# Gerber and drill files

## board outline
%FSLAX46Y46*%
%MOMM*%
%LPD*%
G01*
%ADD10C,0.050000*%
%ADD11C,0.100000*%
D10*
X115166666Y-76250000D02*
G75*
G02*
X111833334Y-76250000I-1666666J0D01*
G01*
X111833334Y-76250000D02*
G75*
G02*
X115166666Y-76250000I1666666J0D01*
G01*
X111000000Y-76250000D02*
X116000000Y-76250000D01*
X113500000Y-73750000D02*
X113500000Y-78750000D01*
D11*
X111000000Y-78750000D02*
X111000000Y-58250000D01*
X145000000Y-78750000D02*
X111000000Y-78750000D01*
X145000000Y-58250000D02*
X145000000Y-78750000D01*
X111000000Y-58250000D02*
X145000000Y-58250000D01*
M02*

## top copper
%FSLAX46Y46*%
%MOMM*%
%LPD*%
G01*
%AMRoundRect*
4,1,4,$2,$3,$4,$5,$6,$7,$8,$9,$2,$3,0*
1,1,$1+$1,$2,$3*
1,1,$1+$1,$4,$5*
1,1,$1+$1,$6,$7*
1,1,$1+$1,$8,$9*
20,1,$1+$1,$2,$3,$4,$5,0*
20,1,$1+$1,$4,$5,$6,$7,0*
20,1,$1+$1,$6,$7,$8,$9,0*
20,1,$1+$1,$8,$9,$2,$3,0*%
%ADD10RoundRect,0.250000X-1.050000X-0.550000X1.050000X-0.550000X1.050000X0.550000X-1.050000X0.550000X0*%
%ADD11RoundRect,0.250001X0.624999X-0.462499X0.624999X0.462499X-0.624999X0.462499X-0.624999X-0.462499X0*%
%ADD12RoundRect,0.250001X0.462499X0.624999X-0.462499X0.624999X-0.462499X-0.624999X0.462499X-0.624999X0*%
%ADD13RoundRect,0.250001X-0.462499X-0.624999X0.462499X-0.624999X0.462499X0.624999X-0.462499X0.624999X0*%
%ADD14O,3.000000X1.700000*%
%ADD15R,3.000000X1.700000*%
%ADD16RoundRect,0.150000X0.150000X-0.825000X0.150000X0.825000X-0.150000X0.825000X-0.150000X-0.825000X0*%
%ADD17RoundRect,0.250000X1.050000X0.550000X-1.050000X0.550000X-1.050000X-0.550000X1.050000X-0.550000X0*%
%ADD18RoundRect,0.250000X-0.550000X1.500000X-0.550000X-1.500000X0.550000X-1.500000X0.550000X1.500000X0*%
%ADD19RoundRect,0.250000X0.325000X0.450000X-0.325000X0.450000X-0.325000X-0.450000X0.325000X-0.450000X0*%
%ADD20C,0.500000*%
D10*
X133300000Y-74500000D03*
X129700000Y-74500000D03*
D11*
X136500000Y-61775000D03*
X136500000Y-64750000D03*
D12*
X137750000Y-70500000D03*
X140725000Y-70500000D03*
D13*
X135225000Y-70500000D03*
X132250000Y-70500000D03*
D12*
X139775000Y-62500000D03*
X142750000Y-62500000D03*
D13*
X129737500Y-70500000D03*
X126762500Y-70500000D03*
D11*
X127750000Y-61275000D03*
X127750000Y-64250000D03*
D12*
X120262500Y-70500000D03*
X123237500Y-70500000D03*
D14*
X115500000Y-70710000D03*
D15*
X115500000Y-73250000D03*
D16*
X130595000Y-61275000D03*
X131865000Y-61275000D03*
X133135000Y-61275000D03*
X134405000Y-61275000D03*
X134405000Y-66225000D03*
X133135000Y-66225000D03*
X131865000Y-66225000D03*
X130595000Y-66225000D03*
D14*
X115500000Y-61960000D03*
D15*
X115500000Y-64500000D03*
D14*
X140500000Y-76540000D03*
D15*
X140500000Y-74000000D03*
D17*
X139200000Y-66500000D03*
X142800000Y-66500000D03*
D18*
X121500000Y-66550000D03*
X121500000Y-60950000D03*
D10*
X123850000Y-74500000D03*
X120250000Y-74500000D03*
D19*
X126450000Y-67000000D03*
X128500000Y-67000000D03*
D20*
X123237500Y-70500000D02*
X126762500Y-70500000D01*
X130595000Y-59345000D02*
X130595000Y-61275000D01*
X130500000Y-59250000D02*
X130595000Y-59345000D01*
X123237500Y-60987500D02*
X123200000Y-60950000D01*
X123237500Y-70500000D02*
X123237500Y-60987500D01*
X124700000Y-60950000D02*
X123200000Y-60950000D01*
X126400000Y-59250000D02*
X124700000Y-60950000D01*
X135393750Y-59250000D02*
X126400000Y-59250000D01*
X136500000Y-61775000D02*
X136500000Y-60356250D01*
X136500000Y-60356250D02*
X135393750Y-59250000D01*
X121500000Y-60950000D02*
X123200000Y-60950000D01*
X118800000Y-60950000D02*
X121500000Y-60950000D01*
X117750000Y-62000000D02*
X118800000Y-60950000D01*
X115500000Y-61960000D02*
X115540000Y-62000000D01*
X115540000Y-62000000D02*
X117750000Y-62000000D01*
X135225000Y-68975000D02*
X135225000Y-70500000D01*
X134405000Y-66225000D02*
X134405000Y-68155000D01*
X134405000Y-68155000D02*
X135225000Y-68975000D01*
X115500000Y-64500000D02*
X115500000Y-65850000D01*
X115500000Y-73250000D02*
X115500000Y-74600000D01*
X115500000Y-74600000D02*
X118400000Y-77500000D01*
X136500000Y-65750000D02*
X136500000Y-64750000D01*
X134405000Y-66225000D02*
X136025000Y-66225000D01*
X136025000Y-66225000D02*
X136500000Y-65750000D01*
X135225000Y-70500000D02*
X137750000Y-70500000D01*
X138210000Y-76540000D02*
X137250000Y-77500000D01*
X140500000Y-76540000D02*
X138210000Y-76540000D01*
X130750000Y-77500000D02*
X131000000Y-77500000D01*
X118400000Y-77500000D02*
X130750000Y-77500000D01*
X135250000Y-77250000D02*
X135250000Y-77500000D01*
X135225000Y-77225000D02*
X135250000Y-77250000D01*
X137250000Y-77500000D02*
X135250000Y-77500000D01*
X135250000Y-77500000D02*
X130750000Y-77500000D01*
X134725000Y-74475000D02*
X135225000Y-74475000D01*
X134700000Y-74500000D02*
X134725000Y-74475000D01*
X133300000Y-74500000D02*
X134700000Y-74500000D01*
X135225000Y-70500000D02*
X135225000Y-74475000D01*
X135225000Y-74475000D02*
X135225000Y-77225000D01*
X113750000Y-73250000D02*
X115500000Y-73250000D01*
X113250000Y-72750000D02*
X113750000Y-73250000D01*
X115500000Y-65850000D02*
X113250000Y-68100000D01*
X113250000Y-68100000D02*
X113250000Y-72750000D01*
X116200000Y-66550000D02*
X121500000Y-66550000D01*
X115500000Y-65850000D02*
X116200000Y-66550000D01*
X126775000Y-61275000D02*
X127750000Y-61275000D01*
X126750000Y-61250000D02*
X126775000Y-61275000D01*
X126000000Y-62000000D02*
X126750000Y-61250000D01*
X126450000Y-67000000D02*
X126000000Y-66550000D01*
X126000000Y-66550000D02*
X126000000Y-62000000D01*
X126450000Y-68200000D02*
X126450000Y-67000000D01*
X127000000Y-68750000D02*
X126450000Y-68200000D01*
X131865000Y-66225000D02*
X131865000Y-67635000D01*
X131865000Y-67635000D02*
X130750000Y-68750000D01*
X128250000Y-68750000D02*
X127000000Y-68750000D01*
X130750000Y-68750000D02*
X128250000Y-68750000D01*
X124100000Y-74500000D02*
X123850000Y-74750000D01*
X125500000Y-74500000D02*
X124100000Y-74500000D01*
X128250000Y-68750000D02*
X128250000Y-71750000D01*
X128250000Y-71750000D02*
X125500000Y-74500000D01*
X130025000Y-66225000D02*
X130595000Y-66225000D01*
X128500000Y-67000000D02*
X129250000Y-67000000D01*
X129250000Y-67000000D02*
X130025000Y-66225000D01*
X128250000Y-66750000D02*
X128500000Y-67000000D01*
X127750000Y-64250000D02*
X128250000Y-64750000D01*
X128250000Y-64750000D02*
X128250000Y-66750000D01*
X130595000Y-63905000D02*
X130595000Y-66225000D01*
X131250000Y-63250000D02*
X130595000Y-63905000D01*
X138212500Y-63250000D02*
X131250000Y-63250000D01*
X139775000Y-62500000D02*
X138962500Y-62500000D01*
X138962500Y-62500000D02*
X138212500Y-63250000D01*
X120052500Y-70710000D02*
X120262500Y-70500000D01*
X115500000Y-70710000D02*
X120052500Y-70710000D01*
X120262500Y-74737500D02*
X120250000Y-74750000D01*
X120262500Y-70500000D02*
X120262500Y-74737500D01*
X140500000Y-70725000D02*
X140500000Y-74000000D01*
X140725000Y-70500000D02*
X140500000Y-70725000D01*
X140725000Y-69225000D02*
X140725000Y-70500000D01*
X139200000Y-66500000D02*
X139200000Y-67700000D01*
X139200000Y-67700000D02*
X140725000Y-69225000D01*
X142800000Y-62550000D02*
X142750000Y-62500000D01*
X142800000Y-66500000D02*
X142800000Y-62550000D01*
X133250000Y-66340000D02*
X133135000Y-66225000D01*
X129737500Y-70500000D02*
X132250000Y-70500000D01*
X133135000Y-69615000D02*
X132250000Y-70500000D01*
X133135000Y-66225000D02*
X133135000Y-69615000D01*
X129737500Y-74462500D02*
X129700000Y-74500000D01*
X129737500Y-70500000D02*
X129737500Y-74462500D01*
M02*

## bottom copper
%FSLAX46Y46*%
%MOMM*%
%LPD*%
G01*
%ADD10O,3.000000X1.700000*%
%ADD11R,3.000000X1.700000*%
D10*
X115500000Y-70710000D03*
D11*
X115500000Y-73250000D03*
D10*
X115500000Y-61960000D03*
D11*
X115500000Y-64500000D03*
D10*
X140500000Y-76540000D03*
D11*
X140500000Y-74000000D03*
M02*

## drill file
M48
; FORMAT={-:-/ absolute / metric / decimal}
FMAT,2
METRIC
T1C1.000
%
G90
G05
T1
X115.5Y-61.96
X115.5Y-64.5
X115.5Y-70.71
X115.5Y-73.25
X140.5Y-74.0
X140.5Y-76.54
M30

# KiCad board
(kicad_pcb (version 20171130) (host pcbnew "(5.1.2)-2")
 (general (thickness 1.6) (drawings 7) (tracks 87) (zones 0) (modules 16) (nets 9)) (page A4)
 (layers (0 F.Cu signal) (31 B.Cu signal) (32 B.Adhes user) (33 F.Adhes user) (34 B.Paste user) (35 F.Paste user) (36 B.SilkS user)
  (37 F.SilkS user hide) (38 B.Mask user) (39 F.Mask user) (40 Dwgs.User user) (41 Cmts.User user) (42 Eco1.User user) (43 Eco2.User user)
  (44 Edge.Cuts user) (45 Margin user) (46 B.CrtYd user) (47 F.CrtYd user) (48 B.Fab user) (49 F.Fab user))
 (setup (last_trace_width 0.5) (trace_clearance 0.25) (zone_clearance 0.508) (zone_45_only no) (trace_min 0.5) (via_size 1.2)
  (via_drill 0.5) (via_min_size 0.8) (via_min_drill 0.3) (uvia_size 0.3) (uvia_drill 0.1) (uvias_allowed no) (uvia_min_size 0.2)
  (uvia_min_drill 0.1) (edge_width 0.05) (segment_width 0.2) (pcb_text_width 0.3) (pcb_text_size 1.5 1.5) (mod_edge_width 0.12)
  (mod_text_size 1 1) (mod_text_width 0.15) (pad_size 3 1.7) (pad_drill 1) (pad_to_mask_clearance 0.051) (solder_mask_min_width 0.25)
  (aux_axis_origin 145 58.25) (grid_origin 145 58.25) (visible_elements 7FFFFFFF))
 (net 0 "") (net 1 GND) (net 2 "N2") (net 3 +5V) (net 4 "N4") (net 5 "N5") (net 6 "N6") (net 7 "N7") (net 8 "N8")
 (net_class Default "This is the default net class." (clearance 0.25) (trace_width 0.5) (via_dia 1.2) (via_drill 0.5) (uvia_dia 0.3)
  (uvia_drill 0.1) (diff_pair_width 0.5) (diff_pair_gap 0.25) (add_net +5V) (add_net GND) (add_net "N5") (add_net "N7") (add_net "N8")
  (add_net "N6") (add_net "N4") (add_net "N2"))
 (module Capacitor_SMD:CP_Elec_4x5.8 (layer F.Cu) (at 131.5 74.5)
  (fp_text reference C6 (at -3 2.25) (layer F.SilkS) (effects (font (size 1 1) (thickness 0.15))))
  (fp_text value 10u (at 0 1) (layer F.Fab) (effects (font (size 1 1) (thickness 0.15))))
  (pad 2 smd roundrect (at 1.8 0) (size 2.6 1.6) (layers F.Cu F.Paste F.Mask) (roundrect_rratio 0.15625) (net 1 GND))
  (pad 1 smd roundrect (at -1.8 0) (size 2.6 1.6) (layers F.Cu F.Paste F.Mask) (roundrect_rratio 0.15625) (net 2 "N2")))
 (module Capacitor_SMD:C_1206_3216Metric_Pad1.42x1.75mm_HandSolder (layer F.Cu) (at 136.5 63.2625 90)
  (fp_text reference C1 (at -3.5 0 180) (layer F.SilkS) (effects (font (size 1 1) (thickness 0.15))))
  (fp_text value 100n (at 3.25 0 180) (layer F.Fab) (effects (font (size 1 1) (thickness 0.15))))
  (pad 2 smd roundrect (at 1.4875 0 90) (size 1.425 1.75) (layers F.Cu F.Paste F.Mask) (roundrect_rratio 0.175439) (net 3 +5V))
  (pad 1 smd roundrect (at -1.4875 0 90) (size 1.425 1.75) (layers F.Cu F.Paste F.Mask) (roundrect_rratio 0.175439) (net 1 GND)))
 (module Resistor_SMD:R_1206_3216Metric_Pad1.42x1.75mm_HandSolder (layer F.Cu) (at 139.2375 70.5 180)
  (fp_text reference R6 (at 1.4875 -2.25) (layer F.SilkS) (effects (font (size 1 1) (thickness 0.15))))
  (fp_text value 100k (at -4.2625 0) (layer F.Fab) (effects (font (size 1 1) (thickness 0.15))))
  (pad 2 smd roundrect (at 1.4875 0 180) (size 1.425 1.75) (layers F.Cu F.Paste F.Mask) (roundrect_rratio 0.175439) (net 1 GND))
  (pad 1 smd roundrect (at -1.4875 0 180) (size 1.425 1.75) (layers F.Cu F.Paste F.Mask) (roundrect_rratio 0.175439) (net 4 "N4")))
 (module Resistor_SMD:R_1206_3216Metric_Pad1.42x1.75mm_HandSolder (layer F.Cu) (at 133.7375 70.5)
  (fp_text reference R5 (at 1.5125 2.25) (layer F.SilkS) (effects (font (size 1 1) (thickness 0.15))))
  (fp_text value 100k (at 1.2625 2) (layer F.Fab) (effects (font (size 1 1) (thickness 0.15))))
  (pad 2 smd roundrect (at 1.4875 0) (size 1.425 1.75) (layers F.Cu F.Paste F.Mask) (roundrect_rratio 0.175439) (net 1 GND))
  (pad 1 smd roundrect (at -1.4875 0) (size 1.425 1.75) (layers F.Cu F.Paste F.Mask) (roundrect_rratio 0.175439) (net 2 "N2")))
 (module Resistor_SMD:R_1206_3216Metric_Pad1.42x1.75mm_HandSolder (layer F.Cu) (at 141.2625 62.5 180)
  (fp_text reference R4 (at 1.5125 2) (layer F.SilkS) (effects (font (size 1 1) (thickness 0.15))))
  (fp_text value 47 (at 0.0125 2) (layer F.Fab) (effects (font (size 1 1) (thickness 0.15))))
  (pad 2 smd roundrect (at 1.4875 0 180) (size 1.425 1.75) (layers F.Cu F.Paste F.Mask) (roundrect_rratio 0.175439) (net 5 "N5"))
  (pad 1 smd roundrect (at -1.4875 0 180) (size 1.425 1.75) (layers F.Cu F.Paste F.Mask) (roundrect_rratio 0.175439) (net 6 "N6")))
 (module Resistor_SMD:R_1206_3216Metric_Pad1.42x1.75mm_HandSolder (layer F.Cu) (at 128.25 70.5)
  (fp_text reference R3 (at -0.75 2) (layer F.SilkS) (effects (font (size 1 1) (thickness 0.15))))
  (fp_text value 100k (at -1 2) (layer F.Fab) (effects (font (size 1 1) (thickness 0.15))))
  (pad 2 smd roundrect (at 1.4875 0) (size 1.425 1.75) (layers F.Cu F.Paste F.Mask) (roundrect_rratio 0.175439) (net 2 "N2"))
  (pad 1 smd roundrect (at -1.4875 0) (size 1.425 1.75) (layers F.Cu F.Paste F.Mask) (roundrect_rratio 0.175439) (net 3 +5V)))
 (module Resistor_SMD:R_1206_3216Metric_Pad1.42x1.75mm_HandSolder (layer F.Cu) (at 127.75 62.7625 90)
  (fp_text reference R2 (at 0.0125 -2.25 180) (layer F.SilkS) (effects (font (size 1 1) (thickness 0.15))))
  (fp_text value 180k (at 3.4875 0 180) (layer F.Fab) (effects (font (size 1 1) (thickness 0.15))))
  (pad 2 smd roundrect (at 1.4875 0 90) (size 1.425 1.75) (layers F.Cu F.Paste F.Mask) (roundrect_rratio 0.175439) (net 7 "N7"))
  (pad 1 smd roundrect (at -1.4875 0 90) (size 1.425 1.75) (layers F.Cu F.Paste F.Mask) (roundrect_rratio 0.175439) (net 5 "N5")))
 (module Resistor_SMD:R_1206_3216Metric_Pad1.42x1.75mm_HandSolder (layer F.Cu) (at 121.75 70.5 180)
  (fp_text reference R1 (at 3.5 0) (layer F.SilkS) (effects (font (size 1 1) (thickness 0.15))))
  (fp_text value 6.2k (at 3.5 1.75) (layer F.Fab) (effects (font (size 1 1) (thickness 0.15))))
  (pad 2 smd roundrect (at 1.4875 0 180) (size 1.425 1.75) (layers F.Cu F.Paste F.Mask) (roundrect_rratio 0.175439) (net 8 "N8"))
  (pad 1 smd roundrect (at -1.4875 0 180) (size 1.425 1.75) (layers F.Cu F.Paste F.Mask) (roundrect_rratio 0.175439) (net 3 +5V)))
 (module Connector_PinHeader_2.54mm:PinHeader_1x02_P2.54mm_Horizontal (layer F.Cu) (at 115.5 73.25 180)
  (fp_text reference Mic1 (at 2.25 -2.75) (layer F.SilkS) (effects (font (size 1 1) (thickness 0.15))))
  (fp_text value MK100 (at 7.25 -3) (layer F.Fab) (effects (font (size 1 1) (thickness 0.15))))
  (pad 2 thru_hole oval (at 0 2.54 180) (size 3 1.7) (drill 1) (layers *.Cu *.Mask) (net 8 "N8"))
  (pad 1 thru_hole rect (at 0 0 180) (size 3 1.7) (drill 1) (layers *.Cu *.Mask) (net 1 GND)))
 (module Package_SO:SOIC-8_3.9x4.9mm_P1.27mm (layer F.Cu) (at 132.5 63.75 90)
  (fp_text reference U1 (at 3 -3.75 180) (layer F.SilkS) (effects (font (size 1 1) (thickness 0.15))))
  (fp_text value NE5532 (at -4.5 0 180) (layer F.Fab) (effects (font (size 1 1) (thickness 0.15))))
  (pad 8 smd roundrect (at 2.475 -1.905 90) (size 1.95 0.6) (layers F.Cu F.Paste F.Mask) (roundrect_rratio 0.25) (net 3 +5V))
  (pad 7 smd roundrect (at 2.475 -0.635 90) (size 1.95 0.6) (layers F.Cu F.Paste F.Mask) (roundrect_rratio 0.25))
  (pad 6 smd roundrect (at 2.475 0.635 90) (size 1.95 0.6) (layers F.Cu F.Paste F.Mask) (roundrect_rratio 0.25))
  (pad 5 smd roundrect (at 2.475 1.905 90) (size 1.95 0.6) (layers F.Cu F.Paste F.Mask) (roundrect_rratio 0.25))
  (pad 4 smd roundrect (at -2.475 1.905 90) (size 1.95 0.6) (layers F.Cu F.Paste F.Mask) (roundrect_rratio 0.25) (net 1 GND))
  (pad 3 smd roundrect (at -2.475 0.635 90) (size 1.95 0.6) (layers F.Cu F.Paste F.Mask) (roundrect_rratio 0.25) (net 2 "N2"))
  (pad 2 smd roundrect (at -2.475 -0.635 90) (size 1.95 0.6) (layers F.Cu F.Paste F.Mask) (roundrect_rratio 0.25) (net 7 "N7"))
  (pad 1 smd roundrect (at -2.475 -1.905 90) (size 1.95 0.6) (layers F.Cu F.Paste F.Mask) (roundrect_rratio 0.25) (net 5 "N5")))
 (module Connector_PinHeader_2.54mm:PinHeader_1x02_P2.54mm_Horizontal (layer F.Cu) (at 115.5 64.5 180)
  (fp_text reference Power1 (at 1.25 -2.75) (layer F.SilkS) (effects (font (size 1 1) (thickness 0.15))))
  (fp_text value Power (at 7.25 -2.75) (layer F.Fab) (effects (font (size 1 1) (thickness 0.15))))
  (pad 2 thru_hole oval (at 0 2.54 180) (size 3 1.7) (drill 1) (layers *.Cu *.Mask) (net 3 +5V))
  (pad 1 thru_hole rect (at 0 0 180) (size 3 1.7) (drill 1) (layers *.Cu *.Mask) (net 1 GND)))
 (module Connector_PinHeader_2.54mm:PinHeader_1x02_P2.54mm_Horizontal (layer F.Cu) (at 140.5 74)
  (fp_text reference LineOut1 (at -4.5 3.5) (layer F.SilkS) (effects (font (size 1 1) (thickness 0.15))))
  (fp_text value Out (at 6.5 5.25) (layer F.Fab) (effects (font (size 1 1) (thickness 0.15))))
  (pad 2 thru_hole oval (at 0 2.54) (size 3 1.7) (drill 1) (layers *.Cu *.Mask) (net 1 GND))
  (pad 1 thru_hole rect (at 0 0) (size 3 1.7) (drill 1) (layers *.Cu *.Mask) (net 4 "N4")))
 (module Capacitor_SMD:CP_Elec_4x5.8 (layer F.Cu) (at 141 66.5 180)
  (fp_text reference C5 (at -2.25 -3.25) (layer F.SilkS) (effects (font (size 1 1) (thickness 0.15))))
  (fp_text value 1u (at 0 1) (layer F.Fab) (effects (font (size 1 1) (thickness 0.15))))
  (pad 2 smd roundrect (at 1.8 0 180) (size 2.6 1.6) (layers F.Cu F.Paste F.Mask) (roundrect_rratio 0.15625) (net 4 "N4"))
  (pad 1 smd roundrect (at -1.8 0 180) (size 2.6 1.6) (layers F.Cu F.Paste F.Mask) (roundrect_rratio 0.15625) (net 6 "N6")))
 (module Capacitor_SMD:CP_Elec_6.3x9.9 (layer F.Cu) (at 121.5 63.75 270)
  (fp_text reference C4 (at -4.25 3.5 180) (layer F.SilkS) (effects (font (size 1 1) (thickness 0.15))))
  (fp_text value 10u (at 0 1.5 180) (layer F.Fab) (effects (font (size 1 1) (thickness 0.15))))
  (pad 2 smd roundrect (at 2.8 0 270) (size 3.5 1.6) (layers F.Cu F.Paste F.Mask) (roundrect_rratio 0.15625) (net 1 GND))
  (pad 1 smd roundrect (at -2.8 0 270) (size 3.5 1.6) (layers F.Cu F.Paste F.Mask) (roundrect_rratio 0.15625) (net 3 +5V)))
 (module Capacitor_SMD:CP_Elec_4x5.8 (layer F.Cu) (at 122.05 74.5)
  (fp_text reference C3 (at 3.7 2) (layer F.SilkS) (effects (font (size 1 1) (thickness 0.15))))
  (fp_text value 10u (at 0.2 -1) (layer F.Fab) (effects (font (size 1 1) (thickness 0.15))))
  (pad 2 smd roundrect (at 1.8 0) (size 2.6 1.6) (layers F.Cu F.Paste F.Mask) (roundrect_rratio 0.15625) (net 7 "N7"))
  (pad 1 smd roundrect (at -1.8 0) (size 2.6 1.6) (layers F.Cu F.Paste F.Mask) (roundrect_rratio 0.15625) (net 8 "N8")))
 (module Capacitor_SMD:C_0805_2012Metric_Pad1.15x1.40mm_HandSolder (layer F.Cu) (at 127.475 67 180)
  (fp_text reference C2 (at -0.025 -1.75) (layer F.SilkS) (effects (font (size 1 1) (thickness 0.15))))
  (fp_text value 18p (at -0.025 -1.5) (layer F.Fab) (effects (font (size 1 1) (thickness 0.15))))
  (pad 2 smd roundrect (at 1.025 0 180) (size 1.15 1.4) (layers F.Cu F.Paste F.Mask) (roundrect_rratio 0.217391) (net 7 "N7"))
  (pad 1 smd roundrect (at -1.025 0 180) (size 1.15 1.4) (layers F.Cu F.Paste F.Mask) (roundrect_rratio 0.217391) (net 5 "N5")))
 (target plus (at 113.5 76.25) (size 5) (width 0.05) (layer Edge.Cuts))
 (gr_line (start 111 78.75) (end 111 58.25) (layer Edge.Cuts) (width 0.1))
 (gr_line (start 145 78.75) (end 111 78.75) (layer Edge.Cuts) (width 0.1))
 (gr_line (start 145 58.25) (end 145 78.75) (layer Edge.Cuts) (width 0.1))
 (gr_line (start 111 58.25) (end 145 58.25) (layer Edge.Cuts) (width 0.1))
 (segment (start 123.2375 70.5) (end 126.7625 70.5) (width 0.5) (layer F.Cu) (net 3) (status 30))
 (segment (start 130.595 59.345) (end 130.595 61.275) (width 0.5) (layer F.Cu) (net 3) (status 20))
 (segment (start 130.5 59.25) (end 130.595 59.345) (width 0.5) (layer F.Cu) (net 3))
 (segment (start 123.2375 60.9875) (end 123.2 60.95) (width 0.5) (layer F.Cu) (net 3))
 (segment (start 123.2375 70.5) (end 123.2375 60.9875) (width 0.5) (layer F.Cu) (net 3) (status 10))
 (segment (start 124.7 60.95) (end 123.2 60.95) (width 0.5) (layer F.Cu) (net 3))
 (segment (start 126.4 59.25) (end 124.7 60.95) (width 0.5) (layer F.Cu) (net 3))
 (segment (start 135.39375 59.25) (end 126.4 59.25) (width 0.5) (layer F.Cu) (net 3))
 (segment (start 136.5 61.775) (end 136.5 60.35625) (width 0.5) (layer F.Cu) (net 3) (status 10))
 (segment (start 136.5 60.35625) (end 135.39375 59.25) (width 0.5) (layer F.Cu) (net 3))
 (segment (start 121.5 60.95) (end 123.2 60.95) (width 0.5) (layer F.Cu) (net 3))
 (segment (start 118.8 60.95) (end 121.5 60.95) (width 0.5) (layer F.Cu) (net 3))
 (segment (start 117.75 62) (end 118.8 60.95) (width 0.5) (layer F.Cu) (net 3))
 (segment (start 115.5 61.96) (end 115.54 62) (width 0.5) (layer F.Cu) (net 3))
 (segment (start 115.54 62) (end 117.75 62) (width 0.5) (layer F.Cu) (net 3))
 (segment (start 135.225 68.975) (end 135.225 70.5) (width 0.5) (layer F.Cu) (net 1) (status 20))
 (segment (start 134.405 66.225) (end 134.405 68.155) (width 0.5) (layer F.Cu) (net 1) (status 10))
 (segment (start 134.405 68.155) (end 135.225 68.975) (width 0.5) (layer F.Cu) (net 1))
 (segment (start 115.5 64.5) (end 115.5 65.85) (width 0.5) (layer F.Cu) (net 1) (status 10))
 (segment (start 115.5 73.25) (end 115.5 74.6) (width 0.5) (layer F.Cu) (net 1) (status 10))
 (segment (start 115.5 74.6) (end 118.4 77.5) (width 0.5) (layer F.Cu) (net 1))
 (segment (start 136.5 65.75) (end 136.5 64.75) (width 0.5) (layer F.Cu) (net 1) (status 20))
 (segment (start 134.405 66.225) (end 136.025 66.225) (width 0.5) (layer F.Cu) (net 1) (status 10))
 (segment (start 136.025 66.225) (end 136.5 65.75) (width 0.5) (layer F.Cu) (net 1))
 (segment (start 135.225 70.5) (end 137.75 70.5) (width 0.5) (layer F.Cu) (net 1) (status 30))
 (segment (start 138.21 76.54) (end 137.25 77.5) (width 0.5) (layer F.Cu) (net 1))
 (segment (start 140.5 76.54) (end 138.21 76.54) (width 0.5) (layer F.Cu) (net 1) (status 10))
 (segment (start 130.75 77.5) (end 131 77.5) (width 0.5) (layer F.Cu) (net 1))
 (segment (start 118.4 77.5) (end 130.75 77.5) (width 0.5) (layer F.Cu) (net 1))
 (segment (start 135.25 77.25) (end 135.25 77.5) (width 0.5) (layer F.Cu) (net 1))
 (segment (start 135.225 77.225) (end 135.25 77.25) (width 0.5) (layer F.Cu) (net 1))
 (segment (start 137.25 77.5) (end 135.25 77.5) (width 0.5) (layer F.Cu) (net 1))
 (segment (start 135.25 77.5) (end 130.75 77.5) (width 0.5) (layer F.Cu) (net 1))
 (segment (start 134.725 74.475) (end 135.225 74.475) (width 0.5) (layer F.Cu) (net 1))
 (segment (start 134.7 74.5) (end 134.725 74.475) (width 0.5) (layer F.Cu) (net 1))
 (segment (start 133.3 74.5) (end 134.7 74.5) (width 0.5) (layer F.Cu) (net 1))
 (segment (start 135.225 70.5) (end 135.225 74.475) (width 0.5) (layer F.Cu) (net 1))
 (segment (start 135.225 74.475) (end 135.225 77.225) (width 0.5) (layer F.Cu) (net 1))
 (segment (start 113.75 73.25) (end 115.5 73.25) (width 0.5) (layer F.Cu) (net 1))
 (segment (start 113.25 72.75) (end 113.75 73.25) (width 0.5) (layer F.Cu) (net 1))
 (segment (start 115.5 65.85) (end 113.25 68.1) (width 0.5) (layer F.Cu) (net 1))
 (segment (start 113.25 68.1) (end 113.25 72.75) (width 0.5) (layer F.Cu) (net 1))
 (segment (start 116.2 66.55) (end 121.5 66.55) (width 0.5) (layer F.Cu) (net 1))
 (segment (start 115.5 65.85) (end 116.2 66.55) (width 0.5) (layer F.Cu) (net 1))
 (segment (start 126.775 61.275) (end 127.75 61.275) (width 0.5) (layer F.Cu) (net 7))
 (segment (start 126.75 61.25) (end 126.775 61.275) (width 0.5) (layer F.Cu) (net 7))
 (segment (start 126 62) (end 126.75 61.25) (width 0.5) (layer F.Cu) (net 7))
 (segment (start 126.45 67) (end 126 66.55) (width 0.5) (layer F.Cu) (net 7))
 (segment (start 126 66.55) (end 126 62) (width 0.5) (layer F.Cu) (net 7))
 (segment (start 126.45 68.2) (end 126.45 67) (width 0.5) (layer F.Cu) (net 7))
 (segment (start 127 68.75) (end 126.45 68.2) (width 0.5) (layer F.Cu) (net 7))
 (segment (start 131.865 66.225) (end 131.865 67.635) (width 0.5) (layer F.Cu) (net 7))
 (segment (start 131.865 67.635) (end 130.75 68.75) (width 0.5) (layer F.Cu) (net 7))
 (segment (start 128.25 68.75) (end 127 68.75) (width 0.5) (layer F.Cu) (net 7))
 (segment (start 130.75 68.75) (end 128.25 68.75) (width 0.5) (layer F.Cu) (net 7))
 (segment (start 124.1 74.5) (end 123.85 74.75) (width 0.5) (layer F.Cu) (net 7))
 (segment (start 125.5 74.5) (end 124.1 74.5) (width 0.5) (layer F.Cu) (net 7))
 (segment (start 128.25 68.75) (end 128.25 71.75) (width 0.5) (layer F.Cu) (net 7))
 (segment (start 128.25 71.75) (end 125.5 74.5) (width 0.5) (layer F.Cu) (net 7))
 (segment (start 130.025 66.225) (end 130.595 66.225) (width 0.5) (layer F.Cu) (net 5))
 (segment (start 128.5 67) (end 129.25 67) (width 0.5) (layer F.Cu) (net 5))
 (segment (start 129.25 67) (end 130.025 66.225) (width 0.5) (layer F.Cu) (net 5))
 (segment (start 128.25 66.75) (end 128.5 67) (width 0.5) (layer F.Cu) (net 5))
 (segment (start 127.75 64.25) (end 128.25 64.75) (width 0.5) (layer F.Cu) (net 5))
 (segment (start 128.25 64.75) (end 128.25 66.75) (width 0.5) (layer F.Cu) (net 5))
 (segment (start 130.595 63.905) (end 130.595 66.225) (width 0.5) (layer F.Cu) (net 5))
 (segment (start 131.25 63.25) (end 130.595 63.905) (width 0.5) (layer F.Cu) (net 5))
 (segment (start 138.2125 63.25) (end 131.25 63.25) (width 0.5) (layer F.Cu) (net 5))
 (segment (start 139.775 62.5) (end 138.9625 62.5) (width 0.5) (layer F.Cu) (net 5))
 (segment (start 138.9625 62.5) (end 138.2125 63.25) (width 0.5) (layer F.Cu) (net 5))
 (segment (start 120.0525 70.71) (end 120.2625 70.5) (width 0.5) (layer F.Cu) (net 8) (status 30))
 (segment (start 115.5 70.71) (end 120.0525 70.71) (width 0.5) (layer F.Cu) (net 8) (status 30))
 (segment (start 120.2625 74.7375) (end 120.25 74.75) (width 0.5) (layer F.Cu) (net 8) (status 30))
 (segment (start 120.2625 70.5) (end 120.2625 74.7375) (width 0.5) (layer F.Cu) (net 8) (status 30))
 (segment (start 140.5 70.725) (end 140.5 74) (width 0.5) (layer F.Cu) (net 4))
 (segment (start 140.725 70.5) (end 140.5 70.725) (width 0.5) (layer F.Cu) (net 4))
 (segment (start 140.725 69.225) (end 140.725 70.5) (width 0.5) (layer F.Cu) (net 4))
 (segment (start 139.2 66.5) (end 139.2 67.7) (width 0.5) (layer F.Cu) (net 4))
 (segment (start 139.2 67.7) (end 140.725 69.225) (width 0.5) (layer F.Cu) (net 4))
 (segment (start 142.8 62.55) (end 142.75 62.5) (width 0.5) (layer F.Cu) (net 6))
 (segment (start 142.8 66.5) (end 142.8 62.55) (width 0.5) (layer F.Cu) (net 6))
 (segment (start 133.25 66.34) (end 133.135 66.225) (width 0.5) (layer F.Cu) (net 2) (status 30))
 (segment (start 129.7375 70.5) (end 132.25 70.5) (width 0.5) (layer F.Cu) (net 2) (status 30))
 (segment (start 133.135 69.615) (end 132.25 70.5) (width 0.5) (layer F.Cu) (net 2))
 (segment (start 133.135 66.225) (end 133.135 69.615) (width 0.5) (layer F.Cu) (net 2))
 (segment (start 129.7375 74.4625) (end 129.7 74.5) (width 0.5) (layer F.Cu) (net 2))
 (segment (start 129.7375 70.5) (end 129.7375 74.4625) (width 0.5) (layer F.Cu) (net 2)))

